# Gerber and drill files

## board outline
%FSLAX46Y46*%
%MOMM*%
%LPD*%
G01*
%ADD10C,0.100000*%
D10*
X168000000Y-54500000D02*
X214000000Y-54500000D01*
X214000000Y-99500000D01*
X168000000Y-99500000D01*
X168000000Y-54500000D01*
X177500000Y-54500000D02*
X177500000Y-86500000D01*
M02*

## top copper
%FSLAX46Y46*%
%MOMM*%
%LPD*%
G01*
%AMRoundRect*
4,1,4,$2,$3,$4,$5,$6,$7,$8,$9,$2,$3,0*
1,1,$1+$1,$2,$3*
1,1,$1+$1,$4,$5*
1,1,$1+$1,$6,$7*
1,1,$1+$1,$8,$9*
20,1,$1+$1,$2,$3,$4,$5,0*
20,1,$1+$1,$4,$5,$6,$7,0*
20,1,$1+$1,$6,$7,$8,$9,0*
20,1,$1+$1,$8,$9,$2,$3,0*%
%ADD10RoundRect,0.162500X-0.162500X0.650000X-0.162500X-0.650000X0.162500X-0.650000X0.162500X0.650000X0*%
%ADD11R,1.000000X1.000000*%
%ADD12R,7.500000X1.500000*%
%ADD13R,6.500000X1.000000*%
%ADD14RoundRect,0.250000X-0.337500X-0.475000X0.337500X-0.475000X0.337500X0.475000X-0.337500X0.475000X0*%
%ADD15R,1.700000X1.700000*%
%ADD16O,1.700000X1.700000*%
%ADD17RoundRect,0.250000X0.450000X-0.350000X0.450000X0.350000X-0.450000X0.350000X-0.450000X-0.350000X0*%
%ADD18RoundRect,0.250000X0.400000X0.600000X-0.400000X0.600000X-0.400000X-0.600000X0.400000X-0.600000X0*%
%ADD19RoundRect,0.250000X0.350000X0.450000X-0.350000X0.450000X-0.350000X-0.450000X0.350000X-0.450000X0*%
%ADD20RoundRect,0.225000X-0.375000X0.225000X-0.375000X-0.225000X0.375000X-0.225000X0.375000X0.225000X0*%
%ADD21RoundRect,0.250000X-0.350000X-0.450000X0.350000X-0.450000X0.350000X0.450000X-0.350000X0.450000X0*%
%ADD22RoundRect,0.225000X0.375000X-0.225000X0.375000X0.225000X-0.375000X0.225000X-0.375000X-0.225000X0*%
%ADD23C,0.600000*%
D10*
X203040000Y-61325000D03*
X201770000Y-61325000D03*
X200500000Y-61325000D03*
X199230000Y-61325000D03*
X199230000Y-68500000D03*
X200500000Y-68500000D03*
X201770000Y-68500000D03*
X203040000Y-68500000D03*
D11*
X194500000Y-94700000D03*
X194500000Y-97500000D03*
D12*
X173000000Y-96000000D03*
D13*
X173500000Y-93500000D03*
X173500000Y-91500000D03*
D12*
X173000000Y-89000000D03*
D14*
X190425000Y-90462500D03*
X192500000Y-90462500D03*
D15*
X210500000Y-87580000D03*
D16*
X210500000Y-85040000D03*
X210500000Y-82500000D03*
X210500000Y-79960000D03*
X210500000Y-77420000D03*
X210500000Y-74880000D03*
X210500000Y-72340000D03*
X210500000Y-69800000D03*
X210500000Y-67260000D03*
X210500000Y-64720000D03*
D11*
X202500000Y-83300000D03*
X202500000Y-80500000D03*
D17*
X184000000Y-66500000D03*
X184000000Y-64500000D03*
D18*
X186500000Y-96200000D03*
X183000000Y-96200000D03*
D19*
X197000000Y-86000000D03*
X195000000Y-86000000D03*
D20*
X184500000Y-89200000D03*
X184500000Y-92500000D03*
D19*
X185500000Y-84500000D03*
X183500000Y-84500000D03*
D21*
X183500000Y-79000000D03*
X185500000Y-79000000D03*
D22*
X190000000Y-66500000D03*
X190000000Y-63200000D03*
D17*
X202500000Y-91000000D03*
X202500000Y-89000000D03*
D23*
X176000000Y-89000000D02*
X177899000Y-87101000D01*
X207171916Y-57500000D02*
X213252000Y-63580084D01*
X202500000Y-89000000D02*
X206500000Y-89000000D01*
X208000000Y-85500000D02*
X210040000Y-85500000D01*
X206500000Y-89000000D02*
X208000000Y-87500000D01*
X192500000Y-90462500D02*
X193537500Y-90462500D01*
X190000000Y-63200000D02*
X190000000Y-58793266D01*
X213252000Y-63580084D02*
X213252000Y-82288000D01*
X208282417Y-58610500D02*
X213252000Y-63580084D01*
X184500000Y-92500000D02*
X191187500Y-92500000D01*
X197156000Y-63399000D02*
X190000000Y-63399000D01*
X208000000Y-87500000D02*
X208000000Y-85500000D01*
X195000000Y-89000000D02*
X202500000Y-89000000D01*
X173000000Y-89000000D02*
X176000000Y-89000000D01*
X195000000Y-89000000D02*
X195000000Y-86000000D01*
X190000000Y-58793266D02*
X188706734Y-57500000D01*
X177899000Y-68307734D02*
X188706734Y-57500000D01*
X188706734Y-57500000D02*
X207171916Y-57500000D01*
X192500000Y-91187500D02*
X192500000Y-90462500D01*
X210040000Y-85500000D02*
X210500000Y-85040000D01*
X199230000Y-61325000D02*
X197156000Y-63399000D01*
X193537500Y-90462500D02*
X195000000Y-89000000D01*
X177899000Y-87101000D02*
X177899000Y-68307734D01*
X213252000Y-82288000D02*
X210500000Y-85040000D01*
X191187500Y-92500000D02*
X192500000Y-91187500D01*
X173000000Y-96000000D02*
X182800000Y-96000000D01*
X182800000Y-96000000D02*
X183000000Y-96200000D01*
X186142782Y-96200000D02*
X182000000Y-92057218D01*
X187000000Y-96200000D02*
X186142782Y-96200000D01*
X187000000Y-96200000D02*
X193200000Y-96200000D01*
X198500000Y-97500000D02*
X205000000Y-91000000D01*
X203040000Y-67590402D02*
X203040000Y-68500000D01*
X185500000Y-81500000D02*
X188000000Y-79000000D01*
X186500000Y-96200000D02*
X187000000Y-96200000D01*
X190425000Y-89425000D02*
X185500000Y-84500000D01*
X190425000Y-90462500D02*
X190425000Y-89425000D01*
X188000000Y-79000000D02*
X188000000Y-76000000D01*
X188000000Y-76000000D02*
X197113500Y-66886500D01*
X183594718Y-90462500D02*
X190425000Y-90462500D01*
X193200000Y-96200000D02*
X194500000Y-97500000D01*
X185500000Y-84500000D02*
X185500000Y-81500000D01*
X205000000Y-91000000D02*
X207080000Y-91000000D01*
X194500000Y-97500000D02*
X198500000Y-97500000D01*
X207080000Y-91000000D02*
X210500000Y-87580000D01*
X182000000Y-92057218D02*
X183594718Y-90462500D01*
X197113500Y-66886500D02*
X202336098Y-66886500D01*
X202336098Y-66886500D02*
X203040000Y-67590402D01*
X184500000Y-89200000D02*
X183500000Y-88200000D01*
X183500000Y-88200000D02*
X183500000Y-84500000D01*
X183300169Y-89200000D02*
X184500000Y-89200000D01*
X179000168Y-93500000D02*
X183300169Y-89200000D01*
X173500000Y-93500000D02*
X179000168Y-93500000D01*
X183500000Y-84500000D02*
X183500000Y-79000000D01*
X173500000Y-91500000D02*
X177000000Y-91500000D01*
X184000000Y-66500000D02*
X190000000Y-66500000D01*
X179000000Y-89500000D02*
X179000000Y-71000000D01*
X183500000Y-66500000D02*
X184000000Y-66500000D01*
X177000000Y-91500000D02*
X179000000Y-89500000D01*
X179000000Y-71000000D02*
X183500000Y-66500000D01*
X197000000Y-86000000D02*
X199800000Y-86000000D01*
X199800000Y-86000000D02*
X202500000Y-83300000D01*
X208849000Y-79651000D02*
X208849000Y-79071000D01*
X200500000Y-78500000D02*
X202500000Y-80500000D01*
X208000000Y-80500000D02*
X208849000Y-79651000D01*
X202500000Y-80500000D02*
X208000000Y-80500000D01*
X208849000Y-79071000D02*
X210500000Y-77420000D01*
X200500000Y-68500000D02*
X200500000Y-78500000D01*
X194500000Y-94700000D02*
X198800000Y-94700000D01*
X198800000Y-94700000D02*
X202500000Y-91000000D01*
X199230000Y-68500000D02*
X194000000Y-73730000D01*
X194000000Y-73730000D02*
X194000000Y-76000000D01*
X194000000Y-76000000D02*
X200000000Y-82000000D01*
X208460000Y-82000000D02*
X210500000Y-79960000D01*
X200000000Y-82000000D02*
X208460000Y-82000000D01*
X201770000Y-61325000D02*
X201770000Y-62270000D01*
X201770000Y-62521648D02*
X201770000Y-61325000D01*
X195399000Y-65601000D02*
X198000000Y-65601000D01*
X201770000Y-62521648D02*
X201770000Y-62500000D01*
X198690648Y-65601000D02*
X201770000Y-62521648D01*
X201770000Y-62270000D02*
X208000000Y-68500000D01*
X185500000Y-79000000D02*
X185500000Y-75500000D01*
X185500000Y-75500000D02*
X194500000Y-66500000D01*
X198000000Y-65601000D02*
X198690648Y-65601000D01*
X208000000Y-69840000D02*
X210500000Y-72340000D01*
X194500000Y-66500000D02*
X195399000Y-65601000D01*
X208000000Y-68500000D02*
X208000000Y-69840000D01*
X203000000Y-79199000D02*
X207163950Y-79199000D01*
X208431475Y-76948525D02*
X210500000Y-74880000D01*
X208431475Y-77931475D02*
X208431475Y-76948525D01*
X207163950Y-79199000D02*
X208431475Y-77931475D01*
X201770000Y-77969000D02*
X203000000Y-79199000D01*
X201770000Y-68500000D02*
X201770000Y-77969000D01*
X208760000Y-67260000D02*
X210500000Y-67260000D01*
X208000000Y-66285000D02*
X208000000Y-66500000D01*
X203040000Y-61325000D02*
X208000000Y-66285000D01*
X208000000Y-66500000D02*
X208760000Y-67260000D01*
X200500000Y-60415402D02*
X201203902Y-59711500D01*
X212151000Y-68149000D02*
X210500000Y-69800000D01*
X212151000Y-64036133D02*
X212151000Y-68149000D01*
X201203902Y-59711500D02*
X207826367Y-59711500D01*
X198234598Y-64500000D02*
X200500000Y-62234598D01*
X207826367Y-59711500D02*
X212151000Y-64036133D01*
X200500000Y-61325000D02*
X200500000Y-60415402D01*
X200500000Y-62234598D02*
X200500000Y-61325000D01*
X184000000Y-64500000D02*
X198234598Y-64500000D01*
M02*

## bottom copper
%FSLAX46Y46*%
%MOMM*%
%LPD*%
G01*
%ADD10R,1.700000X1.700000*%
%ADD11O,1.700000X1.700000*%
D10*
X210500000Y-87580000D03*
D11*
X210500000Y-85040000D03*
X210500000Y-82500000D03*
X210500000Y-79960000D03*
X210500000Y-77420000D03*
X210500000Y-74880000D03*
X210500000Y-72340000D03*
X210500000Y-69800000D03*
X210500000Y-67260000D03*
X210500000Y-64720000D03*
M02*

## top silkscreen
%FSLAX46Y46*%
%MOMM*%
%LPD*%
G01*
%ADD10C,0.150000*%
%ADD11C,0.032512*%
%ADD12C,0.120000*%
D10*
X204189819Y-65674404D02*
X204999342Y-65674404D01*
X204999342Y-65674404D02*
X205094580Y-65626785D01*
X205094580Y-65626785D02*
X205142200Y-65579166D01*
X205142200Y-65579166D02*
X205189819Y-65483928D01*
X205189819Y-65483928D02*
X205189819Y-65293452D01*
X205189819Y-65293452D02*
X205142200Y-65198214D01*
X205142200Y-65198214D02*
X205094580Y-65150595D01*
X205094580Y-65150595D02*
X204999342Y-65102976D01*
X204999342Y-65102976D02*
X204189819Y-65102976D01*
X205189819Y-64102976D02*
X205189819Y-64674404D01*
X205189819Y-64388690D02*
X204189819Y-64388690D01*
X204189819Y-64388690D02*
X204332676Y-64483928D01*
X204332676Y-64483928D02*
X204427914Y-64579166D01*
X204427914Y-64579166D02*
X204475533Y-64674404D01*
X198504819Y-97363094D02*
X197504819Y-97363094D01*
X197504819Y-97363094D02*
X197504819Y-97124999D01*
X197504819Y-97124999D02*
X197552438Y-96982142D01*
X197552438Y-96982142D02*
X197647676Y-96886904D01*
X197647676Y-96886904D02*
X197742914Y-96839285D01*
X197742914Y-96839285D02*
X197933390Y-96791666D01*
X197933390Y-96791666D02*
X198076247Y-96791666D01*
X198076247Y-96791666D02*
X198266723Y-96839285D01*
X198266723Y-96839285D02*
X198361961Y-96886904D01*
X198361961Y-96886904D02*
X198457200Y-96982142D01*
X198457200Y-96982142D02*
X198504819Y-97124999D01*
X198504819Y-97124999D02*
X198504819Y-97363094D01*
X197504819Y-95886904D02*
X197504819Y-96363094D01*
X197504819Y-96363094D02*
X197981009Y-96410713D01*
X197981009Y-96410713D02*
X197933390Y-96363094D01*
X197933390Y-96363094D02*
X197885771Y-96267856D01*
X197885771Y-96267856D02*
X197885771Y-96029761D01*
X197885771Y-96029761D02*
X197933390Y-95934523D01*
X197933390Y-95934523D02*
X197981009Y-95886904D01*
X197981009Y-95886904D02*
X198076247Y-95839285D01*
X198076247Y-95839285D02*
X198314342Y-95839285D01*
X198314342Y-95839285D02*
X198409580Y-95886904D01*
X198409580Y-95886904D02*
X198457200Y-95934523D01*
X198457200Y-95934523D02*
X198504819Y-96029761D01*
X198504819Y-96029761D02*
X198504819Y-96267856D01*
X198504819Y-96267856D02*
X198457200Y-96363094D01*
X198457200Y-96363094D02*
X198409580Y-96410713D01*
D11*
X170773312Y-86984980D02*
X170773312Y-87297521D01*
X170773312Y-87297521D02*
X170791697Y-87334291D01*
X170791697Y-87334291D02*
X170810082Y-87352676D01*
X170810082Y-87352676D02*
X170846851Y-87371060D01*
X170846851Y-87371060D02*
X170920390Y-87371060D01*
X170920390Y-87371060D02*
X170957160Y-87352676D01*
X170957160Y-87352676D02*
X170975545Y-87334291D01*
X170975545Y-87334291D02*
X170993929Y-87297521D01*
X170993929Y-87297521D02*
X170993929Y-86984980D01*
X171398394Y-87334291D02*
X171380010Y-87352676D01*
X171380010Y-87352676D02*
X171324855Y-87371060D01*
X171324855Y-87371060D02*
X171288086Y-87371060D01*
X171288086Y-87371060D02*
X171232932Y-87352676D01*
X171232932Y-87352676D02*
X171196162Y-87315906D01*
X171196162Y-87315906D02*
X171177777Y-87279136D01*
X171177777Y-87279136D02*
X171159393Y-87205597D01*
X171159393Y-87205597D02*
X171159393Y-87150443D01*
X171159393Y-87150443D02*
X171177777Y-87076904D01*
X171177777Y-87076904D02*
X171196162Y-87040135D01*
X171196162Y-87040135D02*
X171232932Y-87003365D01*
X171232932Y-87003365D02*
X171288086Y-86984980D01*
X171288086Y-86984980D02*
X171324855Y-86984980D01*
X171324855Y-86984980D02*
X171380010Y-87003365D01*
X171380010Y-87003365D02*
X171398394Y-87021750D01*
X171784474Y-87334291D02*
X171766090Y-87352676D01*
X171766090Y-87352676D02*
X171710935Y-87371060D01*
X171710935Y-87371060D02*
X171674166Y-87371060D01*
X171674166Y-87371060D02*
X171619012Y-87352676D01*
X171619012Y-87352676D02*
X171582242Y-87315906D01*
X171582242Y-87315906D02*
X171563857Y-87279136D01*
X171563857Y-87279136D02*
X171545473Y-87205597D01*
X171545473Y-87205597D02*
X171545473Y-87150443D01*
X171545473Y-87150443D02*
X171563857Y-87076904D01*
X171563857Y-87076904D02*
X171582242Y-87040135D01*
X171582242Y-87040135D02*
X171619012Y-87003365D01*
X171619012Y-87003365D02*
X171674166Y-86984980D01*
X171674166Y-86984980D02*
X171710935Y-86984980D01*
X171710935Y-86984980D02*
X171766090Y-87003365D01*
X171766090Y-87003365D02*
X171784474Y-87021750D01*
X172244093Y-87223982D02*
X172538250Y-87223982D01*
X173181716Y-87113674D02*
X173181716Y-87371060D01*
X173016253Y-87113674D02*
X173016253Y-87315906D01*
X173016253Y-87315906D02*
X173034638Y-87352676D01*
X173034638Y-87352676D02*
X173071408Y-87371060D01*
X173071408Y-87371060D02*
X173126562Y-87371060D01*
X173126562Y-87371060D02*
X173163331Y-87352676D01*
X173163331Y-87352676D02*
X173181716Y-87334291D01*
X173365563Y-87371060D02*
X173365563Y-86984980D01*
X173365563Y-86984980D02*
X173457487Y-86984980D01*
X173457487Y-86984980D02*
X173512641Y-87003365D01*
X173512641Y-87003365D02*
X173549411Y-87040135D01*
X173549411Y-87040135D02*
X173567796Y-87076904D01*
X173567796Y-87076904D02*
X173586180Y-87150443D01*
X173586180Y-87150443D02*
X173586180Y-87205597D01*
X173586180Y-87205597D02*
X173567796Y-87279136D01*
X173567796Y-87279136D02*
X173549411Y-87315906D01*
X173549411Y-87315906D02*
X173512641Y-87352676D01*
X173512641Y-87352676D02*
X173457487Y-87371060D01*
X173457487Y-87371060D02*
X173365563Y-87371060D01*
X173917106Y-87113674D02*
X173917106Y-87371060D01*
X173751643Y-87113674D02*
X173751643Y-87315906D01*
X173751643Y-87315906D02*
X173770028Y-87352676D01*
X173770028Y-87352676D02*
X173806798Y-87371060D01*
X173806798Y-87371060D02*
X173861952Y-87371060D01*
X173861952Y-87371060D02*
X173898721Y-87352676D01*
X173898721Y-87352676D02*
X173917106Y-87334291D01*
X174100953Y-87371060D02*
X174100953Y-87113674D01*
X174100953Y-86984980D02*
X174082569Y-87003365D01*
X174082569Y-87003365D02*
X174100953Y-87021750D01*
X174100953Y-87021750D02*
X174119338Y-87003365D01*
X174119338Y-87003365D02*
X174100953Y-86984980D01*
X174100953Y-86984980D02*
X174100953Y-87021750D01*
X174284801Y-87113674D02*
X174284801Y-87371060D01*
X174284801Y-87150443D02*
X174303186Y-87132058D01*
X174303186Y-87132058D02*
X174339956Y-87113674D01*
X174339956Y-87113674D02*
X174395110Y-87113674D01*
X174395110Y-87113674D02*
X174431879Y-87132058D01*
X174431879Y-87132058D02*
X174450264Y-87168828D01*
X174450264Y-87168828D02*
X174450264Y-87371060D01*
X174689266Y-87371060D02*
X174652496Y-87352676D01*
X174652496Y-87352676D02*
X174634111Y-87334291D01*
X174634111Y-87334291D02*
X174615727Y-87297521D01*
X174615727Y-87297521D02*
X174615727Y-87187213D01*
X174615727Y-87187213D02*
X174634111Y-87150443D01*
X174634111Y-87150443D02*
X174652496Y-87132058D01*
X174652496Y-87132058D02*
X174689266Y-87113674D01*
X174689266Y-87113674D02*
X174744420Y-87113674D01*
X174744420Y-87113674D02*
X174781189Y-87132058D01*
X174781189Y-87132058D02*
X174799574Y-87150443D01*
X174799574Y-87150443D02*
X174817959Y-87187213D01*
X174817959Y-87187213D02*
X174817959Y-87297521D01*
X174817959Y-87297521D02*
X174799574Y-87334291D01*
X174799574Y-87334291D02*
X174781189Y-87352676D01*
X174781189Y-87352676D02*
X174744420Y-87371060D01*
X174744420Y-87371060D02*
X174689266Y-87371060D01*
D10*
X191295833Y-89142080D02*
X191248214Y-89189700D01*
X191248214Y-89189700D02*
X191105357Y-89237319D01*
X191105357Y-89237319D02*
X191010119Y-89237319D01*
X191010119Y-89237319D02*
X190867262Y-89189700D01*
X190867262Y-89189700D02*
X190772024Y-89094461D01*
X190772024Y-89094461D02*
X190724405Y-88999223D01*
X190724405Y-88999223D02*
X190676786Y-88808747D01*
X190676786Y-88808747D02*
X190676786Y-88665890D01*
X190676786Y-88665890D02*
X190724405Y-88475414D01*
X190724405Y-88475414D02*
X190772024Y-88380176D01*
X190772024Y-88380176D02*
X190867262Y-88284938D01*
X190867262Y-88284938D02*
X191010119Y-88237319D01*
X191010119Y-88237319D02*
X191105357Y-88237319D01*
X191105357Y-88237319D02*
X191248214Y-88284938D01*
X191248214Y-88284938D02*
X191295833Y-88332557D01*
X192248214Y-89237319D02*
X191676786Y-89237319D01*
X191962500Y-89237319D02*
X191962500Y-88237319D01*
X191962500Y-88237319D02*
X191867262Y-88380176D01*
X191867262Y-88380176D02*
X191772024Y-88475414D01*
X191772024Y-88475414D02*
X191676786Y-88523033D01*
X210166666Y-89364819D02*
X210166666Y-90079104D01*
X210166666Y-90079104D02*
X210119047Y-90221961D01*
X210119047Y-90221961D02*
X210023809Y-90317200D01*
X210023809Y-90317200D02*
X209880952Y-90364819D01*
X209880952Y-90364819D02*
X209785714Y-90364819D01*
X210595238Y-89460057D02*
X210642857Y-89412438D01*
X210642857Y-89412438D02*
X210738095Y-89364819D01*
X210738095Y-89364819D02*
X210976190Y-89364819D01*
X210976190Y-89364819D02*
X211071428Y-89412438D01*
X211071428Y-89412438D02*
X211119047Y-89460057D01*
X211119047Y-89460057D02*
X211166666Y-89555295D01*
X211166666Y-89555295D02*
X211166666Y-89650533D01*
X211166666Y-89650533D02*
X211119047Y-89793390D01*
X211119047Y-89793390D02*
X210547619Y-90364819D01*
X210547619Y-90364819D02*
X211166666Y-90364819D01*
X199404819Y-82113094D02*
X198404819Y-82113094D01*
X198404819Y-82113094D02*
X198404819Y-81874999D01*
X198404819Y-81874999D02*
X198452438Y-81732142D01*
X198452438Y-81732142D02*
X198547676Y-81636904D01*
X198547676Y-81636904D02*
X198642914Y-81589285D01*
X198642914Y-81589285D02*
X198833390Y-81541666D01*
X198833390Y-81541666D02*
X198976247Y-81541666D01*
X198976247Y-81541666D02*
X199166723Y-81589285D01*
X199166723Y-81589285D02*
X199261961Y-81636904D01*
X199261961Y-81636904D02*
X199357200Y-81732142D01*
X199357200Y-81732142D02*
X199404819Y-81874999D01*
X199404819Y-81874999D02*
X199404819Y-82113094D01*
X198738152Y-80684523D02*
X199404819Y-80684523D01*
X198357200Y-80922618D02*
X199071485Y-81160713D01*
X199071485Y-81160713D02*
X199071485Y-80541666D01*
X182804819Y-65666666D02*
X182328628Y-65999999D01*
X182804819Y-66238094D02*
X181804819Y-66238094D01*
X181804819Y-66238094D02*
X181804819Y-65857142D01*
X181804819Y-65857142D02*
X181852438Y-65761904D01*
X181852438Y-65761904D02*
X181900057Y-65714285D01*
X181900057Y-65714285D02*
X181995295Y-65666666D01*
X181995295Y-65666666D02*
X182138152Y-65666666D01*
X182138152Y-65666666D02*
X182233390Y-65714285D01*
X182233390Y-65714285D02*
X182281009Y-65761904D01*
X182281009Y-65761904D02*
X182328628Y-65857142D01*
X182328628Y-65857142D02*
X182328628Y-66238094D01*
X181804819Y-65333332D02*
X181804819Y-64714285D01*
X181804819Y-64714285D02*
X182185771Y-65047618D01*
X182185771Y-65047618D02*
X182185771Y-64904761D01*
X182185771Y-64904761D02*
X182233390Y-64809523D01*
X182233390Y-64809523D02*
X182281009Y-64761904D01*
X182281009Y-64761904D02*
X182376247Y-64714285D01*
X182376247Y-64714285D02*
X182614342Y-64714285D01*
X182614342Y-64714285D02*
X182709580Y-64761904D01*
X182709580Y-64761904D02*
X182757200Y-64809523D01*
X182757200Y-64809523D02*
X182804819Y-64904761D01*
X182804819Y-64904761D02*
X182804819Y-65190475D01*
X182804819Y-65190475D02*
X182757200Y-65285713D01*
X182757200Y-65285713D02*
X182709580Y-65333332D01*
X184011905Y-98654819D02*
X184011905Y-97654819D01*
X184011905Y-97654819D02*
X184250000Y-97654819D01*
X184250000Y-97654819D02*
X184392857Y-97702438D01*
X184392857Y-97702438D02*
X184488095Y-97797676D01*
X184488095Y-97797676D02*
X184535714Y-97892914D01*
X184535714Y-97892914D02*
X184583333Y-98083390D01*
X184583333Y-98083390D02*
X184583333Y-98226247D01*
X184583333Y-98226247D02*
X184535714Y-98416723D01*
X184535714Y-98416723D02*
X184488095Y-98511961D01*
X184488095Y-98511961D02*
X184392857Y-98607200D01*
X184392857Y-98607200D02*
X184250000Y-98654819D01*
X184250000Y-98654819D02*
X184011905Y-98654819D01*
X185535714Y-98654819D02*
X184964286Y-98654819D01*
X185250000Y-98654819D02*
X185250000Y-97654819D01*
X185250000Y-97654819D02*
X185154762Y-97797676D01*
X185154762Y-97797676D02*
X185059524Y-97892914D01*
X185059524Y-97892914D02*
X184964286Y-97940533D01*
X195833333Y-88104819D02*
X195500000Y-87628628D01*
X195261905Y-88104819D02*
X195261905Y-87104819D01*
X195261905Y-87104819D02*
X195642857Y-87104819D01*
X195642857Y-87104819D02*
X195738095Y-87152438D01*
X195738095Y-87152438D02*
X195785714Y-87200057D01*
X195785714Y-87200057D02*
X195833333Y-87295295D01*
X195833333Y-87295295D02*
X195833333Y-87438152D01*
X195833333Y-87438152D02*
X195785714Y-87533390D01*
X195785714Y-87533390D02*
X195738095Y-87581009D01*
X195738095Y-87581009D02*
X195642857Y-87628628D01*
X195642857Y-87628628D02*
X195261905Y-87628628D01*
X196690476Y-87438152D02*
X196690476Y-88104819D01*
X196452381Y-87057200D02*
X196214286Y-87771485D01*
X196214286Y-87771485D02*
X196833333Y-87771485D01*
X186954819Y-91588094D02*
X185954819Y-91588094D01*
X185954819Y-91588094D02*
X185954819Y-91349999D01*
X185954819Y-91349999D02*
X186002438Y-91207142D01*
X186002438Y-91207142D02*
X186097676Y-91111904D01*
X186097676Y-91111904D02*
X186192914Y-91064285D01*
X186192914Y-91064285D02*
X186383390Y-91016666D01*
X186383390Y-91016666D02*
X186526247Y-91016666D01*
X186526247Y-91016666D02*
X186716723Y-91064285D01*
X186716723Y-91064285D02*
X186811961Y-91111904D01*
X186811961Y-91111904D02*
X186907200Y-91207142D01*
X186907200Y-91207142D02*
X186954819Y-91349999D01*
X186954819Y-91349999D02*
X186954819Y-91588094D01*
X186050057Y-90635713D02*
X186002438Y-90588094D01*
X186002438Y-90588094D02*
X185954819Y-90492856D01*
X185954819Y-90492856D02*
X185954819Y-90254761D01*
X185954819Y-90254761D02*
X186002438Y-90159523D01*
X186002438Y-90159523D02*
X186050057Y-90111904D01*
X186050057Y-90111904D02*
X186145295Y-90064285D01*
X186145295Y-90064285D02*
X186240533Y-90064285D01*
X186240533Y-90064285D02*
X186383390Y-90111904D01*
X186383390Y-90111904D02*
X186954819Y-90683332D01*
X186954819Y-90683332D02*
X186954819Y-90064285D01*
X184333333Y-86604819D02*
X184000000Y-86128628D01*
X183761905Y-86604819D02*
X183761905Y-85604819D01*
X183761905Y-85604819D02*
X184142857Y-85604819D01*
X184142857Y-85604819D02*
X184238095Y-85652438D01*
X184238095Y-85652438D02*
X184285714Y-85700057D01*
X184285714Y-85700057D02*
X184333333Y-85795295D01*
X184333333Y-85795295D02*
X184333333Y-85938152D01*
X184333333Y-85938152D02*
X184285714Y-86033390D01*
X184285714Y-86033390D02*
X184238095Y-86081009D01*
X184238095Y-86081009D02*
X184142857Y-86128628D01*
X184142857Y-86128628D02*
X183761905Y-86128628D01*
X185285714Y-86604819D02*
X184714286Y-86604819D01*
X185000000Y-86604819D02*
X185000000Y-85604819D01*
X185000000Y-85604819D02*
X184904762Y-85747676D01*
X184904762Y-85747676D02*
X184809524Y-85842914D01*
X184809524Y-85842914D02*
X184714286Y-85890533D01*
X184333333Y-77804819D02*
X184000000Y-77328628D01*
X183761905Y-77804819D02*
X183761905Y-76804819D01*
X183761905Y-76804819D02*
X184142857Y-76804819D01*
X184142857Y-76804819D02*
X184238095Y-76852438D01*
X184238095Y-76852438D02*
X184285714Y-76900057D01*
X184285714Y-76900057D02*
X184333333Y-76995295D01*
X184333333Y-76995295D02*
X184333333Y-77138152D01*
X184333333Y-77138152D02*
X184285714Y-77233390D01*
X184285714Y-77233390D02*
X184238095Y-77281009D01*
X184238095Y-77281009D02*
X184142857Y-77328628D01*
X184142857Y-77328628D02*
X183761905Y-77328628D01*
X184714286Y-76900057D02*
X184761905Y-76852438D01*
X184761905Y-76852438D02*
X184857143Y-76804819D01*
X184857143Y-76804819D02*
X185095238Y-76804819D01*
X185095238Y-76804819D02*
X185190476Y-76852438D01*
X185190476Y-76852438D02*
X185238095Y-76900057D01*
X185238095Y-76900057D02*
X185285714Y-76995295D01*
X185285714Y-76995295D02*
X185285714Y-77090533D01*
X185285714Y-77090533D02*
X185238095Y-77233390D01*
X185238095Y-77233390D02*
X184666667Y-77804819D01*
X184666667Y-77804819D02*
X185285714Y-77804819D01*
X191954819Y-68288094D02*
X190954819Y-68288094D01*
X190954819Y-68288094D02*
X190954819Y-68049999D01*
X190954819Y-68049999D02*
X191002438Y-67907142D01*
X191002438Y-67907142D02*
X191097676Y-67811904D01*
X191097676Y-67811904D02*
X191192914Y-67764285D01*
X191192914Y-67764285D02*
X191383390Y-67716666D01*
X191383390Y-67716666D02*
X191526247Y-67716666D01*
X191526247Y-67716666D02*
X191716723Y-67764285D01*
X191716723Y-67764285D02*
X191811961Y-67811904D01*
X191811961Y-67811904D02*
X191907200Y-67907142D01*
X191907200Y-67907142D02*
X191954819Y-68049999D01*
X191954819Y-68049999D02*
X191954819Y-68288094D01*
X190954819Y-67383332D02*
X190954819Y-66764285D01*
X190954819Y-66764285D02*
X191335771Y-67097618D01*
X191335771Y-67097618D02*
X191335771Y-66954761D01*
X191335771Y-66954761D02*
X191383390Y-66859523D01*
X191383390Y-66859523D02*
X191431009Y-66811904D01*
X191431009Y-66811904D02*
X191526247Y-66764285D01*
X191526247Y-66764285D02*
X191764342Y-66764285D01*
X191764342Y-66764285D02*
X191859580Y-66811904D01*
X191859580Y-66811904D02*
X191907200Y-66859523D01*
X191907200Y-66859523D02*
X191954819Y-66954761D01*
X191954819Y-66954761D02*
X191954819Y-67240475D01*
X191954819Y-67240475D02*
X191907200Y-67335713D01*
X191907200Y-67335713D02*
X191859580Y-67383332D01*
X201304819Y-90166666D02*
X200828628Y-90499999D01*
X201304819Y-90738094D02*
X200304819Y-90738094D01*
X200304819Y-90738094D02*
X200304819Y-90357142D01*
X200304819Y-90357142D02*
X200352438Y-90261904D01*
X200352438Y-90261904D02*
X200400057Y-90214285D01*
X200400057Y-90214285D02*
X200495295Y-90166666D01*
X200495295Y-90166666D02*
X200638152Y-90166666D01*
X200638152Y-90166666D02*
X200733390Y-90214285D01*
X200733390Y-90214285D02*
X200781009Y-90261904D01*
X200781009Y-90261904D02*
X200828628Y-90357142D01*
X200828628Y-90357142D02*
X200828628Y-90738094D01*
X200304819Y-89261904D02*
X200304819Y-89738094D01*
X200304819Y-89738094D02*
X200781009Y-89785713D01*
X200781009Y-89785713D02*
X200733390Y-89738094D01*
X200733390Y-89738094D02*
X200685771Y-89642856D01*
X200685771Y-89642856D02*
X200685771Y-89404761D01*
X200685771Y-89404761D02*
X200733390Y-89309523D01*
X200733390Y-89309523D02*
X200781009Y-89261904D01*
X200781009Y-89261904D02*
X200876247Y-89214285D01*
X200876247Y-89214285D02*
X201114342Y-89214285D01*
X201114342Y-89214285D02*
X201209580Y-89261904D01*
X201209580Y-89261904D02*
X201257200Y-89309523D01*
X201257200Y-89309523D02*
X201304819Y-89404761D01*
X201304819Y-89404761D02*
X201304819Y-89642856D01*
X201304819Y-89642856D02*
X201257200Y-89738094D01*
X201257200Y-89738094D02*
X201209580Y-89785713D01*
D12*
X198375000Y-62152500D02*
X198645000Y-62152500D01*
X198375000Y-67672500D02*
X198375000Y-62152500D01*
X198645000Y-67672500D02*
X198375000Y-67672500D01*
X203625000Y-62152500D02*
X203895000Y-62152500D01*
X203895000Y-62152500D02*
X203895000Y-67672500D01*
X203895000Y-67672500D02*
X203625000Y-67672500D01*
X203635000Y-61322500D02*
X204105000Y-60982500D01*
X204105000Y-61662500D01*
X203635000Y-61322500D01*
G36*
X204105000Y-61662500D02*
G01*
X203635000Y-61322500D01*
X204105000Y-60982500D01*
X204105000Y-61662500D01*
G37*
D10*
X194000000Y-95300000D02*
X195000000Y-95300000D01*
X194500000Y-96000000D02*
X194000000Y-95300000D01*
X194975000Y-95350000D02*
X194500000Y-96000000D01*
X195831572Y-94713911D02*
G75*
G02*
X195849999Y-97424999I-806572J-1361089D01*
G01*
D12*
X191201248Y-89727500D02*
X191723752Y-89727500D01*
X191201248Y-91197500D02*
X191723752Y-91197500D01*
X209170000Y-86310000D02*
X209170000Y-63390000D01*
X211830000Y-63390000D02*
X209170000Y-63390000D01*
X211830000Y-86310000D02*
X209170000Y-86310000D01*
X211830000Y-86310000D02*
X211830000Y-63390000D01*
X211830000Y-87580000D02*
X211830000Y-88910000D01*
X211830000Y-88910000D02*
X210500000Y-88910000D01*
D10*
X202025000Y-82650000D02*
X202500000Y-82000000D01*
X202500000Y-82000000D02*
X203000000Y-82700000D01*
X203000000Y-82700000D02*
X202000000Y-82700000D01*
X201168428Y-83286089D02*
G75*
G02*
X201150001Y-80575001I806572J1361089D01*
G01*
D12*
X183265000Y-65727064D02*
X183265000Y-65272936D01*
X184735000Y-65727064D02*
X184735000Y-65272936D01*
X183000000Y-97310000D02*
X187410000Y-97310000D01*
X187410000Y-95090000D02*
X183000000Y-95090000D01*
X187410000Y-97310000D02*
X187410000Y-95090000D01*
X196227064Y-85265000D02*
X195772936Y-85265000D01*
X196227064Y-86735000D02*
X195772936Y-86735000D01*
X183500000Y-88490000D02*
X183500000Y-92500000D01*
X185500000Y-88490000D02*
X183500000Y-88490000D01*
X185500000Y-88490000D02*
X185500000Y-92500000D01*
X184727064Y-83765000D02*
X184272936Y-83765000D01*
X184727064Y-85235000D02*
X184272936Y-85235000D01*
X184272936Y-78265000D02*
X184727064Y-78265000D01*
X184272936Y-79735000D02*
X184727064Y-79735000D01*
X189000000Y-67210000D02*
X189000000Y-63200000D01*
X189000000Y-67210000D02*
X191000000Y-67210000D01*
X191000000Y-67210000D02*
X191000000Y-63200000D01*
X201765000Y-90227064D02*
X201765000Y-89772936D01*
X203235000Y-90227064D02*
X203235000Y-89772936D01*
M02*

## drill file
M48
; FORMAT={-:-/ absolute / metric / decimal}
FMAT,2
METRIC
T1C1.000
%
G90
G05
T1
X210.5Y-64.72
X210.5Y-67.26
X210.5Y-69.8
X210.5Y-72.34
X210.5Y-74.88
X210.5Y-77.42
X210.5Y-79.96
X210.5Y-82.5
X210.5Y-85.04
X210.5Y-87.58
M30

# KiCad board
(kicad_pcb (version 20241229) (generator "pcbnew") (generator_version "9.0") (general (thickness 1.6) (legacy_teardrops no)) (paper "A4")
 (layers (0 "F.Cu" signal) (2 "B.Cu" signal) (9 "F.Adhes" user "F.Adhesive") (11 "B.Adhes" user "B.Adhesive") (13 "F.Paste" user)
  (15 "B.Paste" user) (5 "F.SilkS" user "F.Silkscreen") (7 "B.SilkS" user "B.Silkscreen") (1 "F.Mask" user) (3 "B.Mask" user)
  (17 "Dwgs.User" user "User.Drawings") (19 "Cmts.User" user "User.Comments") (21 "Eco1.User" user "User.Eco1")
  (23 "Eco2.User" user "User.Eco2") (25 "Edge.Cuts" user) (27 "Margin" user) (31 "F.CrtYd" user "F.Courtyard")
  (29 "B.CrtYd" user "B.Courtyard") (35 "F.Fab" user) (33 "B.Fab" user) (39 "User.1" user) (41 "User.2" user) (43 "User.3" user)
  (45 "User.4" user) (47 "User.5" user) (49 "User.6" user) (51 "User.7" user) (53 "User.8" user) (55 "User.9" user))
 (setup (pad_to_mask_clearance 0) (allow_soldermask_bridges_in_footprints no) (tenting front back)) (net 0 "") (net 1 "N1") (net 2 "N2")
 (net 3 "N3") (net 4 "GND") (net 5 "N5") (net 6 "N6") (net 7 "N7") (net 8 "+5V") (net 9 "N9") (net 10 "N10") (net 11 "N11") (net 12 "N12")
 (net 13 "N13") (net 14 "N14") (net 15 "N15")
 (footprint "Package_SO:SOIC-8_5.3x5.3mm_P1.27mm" (layer "F.Cu") (at 201.135 64.9125 -90)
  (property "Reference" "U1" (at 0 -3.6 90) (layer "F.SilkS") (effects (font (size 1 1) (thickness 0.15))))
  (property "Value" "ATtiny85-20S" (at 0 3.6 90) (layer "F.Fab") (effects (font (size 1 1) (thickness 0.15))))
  (fp_line (start -2.76 2.76) (end -2.76 2.49) (stroke (width 0.12) (type solid)) (layer "F.SilkS"))
  (fp_line (start 2.76 2.76) (end -2.76 2.76) (stroke (width 0.12) (type solid)) (layer "F.SilkS"))
  (fp_line (start 2.76 2.49) (end 2.76 2.76) (stroke (width 0.12) (type solid)) (layer "F.SilkS"))
  (fp_line (start -2.76 -2.49) (end -2.76 -2.76) (stroke (width 0.12) (type solid)) (layer "F.SilkS"))
  (fp_line (start -2.76 -2.76) (end 2.76 -2.76) (stroke (width 0.12) (type solid)) (layer "F.SilkS"))
  (fp_line (start 2.76 -2.76) (end 2.76 -2.49) (stroke (width 0.12) (type solid)) (layer "F.SilkS"))
  (fp_poly (pts (xy -3.59 -2.5) (xy -3.93 -2.97) (xy -3.25 -2.97)) (stroke (width 0.12) (type solid)) (fill yes) (layer "F.SilkS"))
  (pad "1" smd roundrect (at -3.5875 -1.905 270) (size 1.625 0.65) (layers "F.Cu" "F.Mask" "F.Paste") (roundrect_rratio 0.25) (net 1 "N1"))
  (pad "2" smd roundrect (at -3.5875 -0.635 270) (size 1.625 0.65) (layers "F.Cu" "F.Mask" "F.Paste") (roundrect_rratio 0.25) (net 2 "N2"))
  (pad "3" smd roundrect (at -3.5875 0.635 270) (size 1.625 0.65) (layers "F.Cu" "F.Mask" "F.Paste") (roundrect_rratio 0.25) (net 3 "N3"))
  (pad "4" smd roundrect (at -3.5875 1.905 270) (size 1.625 0.65) (layers "F.Cu" "F.Mask" "F.Paste") (roundrect_rratio 0.25) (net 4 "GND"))
  (pad "5" smd roundrect (at 3.5875 1.905 270) (size 1.625 0.65) (layers "F.Cu" "F.Mask" "F.Paste") (roundrect_rratio 0.25) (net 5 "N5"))
  (pad "6" smd roundrect (at 3.5875 0.635 270) (size 1.625 0.65) (layers "F.Cu" "F.Mask" "F.Paste") (roundrect_rratio 0.25) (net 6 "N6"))
  (pad "7" smd roundrect (at 3.5875 -0.635 270) (size 1.625 0.65) (layers "F.Cu" "F.Mask" "F.Paste") (roundrect_rratio 0.25) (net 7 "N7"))
  (pad "8" smd roundrect (at 3.5875 -1.905 270) (size 1.625 0.65) (layers "F.Cu" "F.Mask" "F.Paste") (roundrect_rratio 0.25) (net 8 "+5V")))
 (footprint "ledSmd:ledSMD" (layer "F.Cu") (at 194.5 96.5 -90)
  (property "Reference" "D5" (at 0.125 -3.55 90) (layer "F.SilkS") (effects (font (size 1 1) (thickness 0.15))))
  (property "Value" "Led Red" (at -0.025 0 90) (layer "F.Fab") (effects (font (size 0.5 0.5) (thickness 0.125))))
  (fp_line (start -1.2 0.5) (end -1.2 -0.5) (stroke (width 0.15) (type solid)) (layer "F.SilkS"))
  (fp_line (start -0.5 0) (end -1.2 0.5) (stroke (width 0.15) (type solid)) (layer "F.SilkS"))
  (fp_line (start -1.15 -0.475) (end -0.5 0) (stroke (width 0.15) (type solid)) (layer "F.SilkS"))
  (fp_arc (start -1.786089 -1.331572) (mid -0.435753 -2.107089) (end 0.924999 -1.349999) (stroke (width 0.15) (type solid))
   (layer "F.SilkS"))
  (pad "1" smd rect (at -1.8 0 270) (size 1 1) (layers "F.Cu" "F.Mask" "F.Paste") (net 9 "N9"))
  (pad "2" smd rect (at 1 0 270) (size 1 1) (layers "F.Cu" "F.Mask" "F.Paste") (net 8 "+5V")))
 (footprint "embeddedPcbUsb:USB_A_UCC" (layer "F.Cu") (at 173.2 92.5)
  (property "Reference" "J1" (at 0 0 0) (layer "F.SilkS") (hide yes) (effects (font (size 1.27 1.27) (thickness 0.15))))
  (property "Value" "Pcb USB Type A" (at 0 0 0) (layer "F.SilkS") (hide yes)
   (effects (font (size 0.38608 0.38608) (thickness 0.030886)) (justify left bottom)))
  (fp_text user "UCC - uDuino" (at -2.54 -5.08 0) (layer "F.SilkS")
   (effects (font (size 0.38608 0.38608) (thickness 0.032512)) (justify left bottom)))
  (pad "1" smd rect (at -0.2 3.5) (size 7.5 1.5) (layers "F.Cu" "F.Mask" "F.Paste") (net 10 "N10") (solder_mask_margin 0.1016))
  (pad "2" smd rect (at 0.3 1) (size 6.5 1) (layers "F.Cu" "F.Mask" "F.Paste") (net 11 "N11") (solder_mask_margin 0.1016))
  (pad "3" smd rect (at 0.3 -1) (size 6.5 1) (layers "F.Cu" "F.Mask" "F.Paste") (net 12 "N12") (solder_mask_margin 0.1016))
  (pad "4" smd rect (at -0.2 -3.5) (size 7.5 1.5) (layers "F.Cu" "F.Mask" "F.Paste") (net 4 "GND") (solder_mask_margin 0.1016)))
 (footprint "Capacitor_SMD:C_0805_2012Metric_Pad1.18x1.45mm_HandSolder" (layer "F.Cu") (at 191.4625 90.4625)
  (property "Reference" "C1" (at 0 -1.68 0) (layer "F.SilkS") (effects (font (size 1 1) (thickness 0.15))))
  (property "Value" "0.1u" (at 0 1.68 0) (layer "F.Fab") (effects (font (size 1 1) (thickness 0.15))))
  (fp_line (start -0.261252 -0.735) (end 0.261252 -0.735) (stroke (width 0.12) (type solid)) (layer "F.SilkS"))
  (fp_line (start -0.261252 0.735) (end 0.261252 0.735) (stroke (width 0.12) (type solid)) (layer "F.SilkS"))
  (pad "1" smd roundrect (at -1.0375 0) (size 1.175 1.45) (layers "F.Cu" "F.Mask" "F.Paste") (roundrect_rratio 0.212766) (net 8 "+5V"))
  (pad "2" smd roundrect (at 1.0375 0) (size 1.175 1.45) (layers "F.Cu" "F.Mask" "F.Paste") (roundrect_rratio 0.212766) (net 4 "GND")))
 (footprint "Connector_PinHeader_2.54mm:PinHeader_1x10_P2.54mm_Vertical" (layer "F.Cu") (at 210.5 87.58 180)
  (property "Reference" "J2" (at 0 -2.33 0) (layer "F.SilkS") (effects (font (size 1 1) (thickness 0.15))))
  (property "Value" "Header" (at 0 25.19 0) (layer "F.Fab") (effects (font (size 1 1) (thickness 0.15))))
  (fp_line (start 1.33 1.27) (end 1.33 24.19) (stroke (width 0.12) (type solid)) (layer "F.SilkS"))
  (fp_line (start -1.33 24.19) (end 1.33 24.19) (stroke (width 0.12) (type solid)) (layer "F.SilkS"))
  (fp_line (start -1.33 1.27) (end 1.33 1.27) (stroke (width 0.12) (type solid)) (layer "F.SilkS"))
  (fp_line (start -1.33 1.27) (end -1.33 24.19) (stroke (width 0.12) (type solid)) (layer "F.SilkS"))
  (fp_line (start -1.33 0) (end -1.33 -1.33) (stroke (width 0.12) (type solid)) (layer "F.SilkS"))
  (fp_line (start -1.33 -1.33) (end 0 -1.33) (stroke (width 0.12) (type solid)) (layer "F.SilkS"))
  (pad "1" thru_hole rect (at 0 0 180) (size 1.7 1.7) (drill 1) (layers "*.Cu" "*.Mask") (remove_unused_layers no) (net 8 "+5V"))
  (pad "2" thru_hole oval (at 0 2.54 180) (size 1.7 1.7) (drill 1) (layers "*.Cu" "*.Mask") (remove_unused_layers no) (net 4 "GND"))
  (pad "3" thru_hole oval (at 0 5.08 180) (size 1.7 1.7) (drill 1) (layers "*.Cu" "*.Mask") (remove_unused_layers no) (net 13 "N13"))
  (pad "4" thru_hole oval (at 0 7.62 180) (size 1.7 1.7) (drill 1) (layers "*.Cu" "*.Mask") (remove_unused_layers no) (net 5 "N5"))
  (pad "5" thru_hole oval (at 0 10.16 180) (size 1.7 1.7) (drill 1) (layers "*.Cu" "*.Mask") (remove_unused_layers no) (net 6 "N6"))
  (pad "6" thru_hole oval (at 0 12.7 180) (size 1.7 1.7) (drill 1) (layers "*.Cu" "*.Mask") (remove_unused_layers no) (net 7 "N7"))
  (pad "7" thru_hole oval (at 0 15.24 180) (size 1.7 1.7) (drill 1) (layers "*.Cu" "*.Mask") (remove_unused_layers no) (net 2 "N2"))
  (pad "8" thru_hole oval (at 0 17.78 180) (size 1.7 1.7) (drill 1) (layers "*.Cu" "*.Mask") (remove_unused_layers no) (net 3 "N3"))
  (pad "9" thru_hole oval (at 0 20.32 180) (size 1.7 1.7) (drill 1) (layers "*.Cu" "*.Mask") (remove_unused_layers no) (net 1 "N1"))
  (pad "10" thru_hole oval (at 0 22.86 180) (size 1.7 1.7) (drill 1) (layers "*.Cu" "*.Mask") (remove_unused_layers no) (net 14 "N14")))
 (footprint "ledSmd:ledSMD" (layer "F.Cu") (at 202.5 81.5 90)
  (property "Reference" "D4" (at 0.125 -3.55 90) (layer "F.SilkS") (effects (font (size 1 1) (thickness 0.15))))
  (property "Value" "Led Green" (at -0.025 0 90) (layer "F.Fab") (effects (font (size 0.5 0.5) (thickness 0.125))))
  (fp_line (start -1.15 -0.475) (end -0.5 0) (stroke (width 0.15) (type solid)) (layer "F.SilkS"))
  (fp_line (start -0.5 0) (end -1.2 0.5) (stroke (width 0.15) (type solid)) (layer "F.SilkS"))
  (fp_line (start -1.2 0.5) (end -1.2 -0.5) (stroke (width 0.15) (type solid)) (layer "F.SilkS"))
  (fp_arc (start -1.786089 -1.331572) (mid -0.435753 -2.107089) (end 0.924999 -1.349999) (stroke (width 0.15) (type solid))
   (layer "F.SilkS"))
  (pad "1" smd rect (at -1.8 0 90) (size 1 1) (layers "F.Cu" "F.Mask" "F.Paste") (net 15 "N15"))
  (pad "2" smd rect (at 1 0 90) (size 1 1) (layers "F.Cu" "F.Mask" "F.Paste") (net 6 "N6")))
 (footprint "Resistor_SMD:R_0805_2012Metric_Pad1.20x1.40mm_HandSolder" (layer "F.Cu") (at 184 65.5 90)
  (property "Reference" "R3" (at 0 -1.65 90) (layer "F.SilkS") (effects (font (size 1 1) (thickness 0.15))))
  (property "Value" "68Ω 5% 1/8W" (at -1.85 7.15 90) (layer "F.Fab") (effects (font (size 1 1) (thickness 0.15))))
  (fp_line (start -0.227064 -0.735) (end 0.227064 -0.735) (stroke (width 0.12) (type solid)) (layer "F.SilkS"))
  (fp_line (start -0.227064 0.735) (end 0.227064 0.735) (stroke (width 0.12) (type solid)) (layer "F.SilkS"))
  (pad "1" smd roundrect (at -1 0 90) (size 1.2 1.4) (layers "F.Cu" "F.Mask" "F.Paste") (roundrect_rratio 0.208333) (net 12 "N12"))
  (pad "2" smd roundrect (at 1 0 90) (size 1.2 1.4) (layers "F.Cu" "F.Mask" "F.Paste") (roundrect_rratio 0.208333) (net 3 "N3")))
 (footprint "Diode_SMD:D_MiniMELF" (layer "F.Cu") (at 184.75 96.2 180)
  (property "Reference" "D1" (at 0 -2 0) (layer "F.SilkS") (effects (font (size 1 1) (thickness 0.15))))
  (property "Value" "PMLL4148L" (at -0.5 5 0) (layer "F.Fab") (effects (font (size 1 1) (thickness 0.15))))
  (fp_line (start 1.75 -1.11) (end -2.66 -1.11) (stroke (width 0.12) (type solid)) (layer "F.SilkS"))
  (fp_line (start -2.66 1.11) (end 1.75 1.11) (stroke (width 0.12) (type solid)) (layer "F.SilkS"))
  (fp_line (start -2.66 -1.11) (end -2.66 1.11) (stroke (width 0.12) (type solid)) (layer "F.SilkS"))
  (pad "1" smd roundrect (at -1.75 0 180) (size 1.3 1.7) (layers "F.Cu" "F.Mask" "F.Paste") (roundrect_rratio 0.1923076923) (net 8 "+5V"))
  (pad "2" smd roundrect (at 1.75 0 180) (size 1.3 1.7) (layers "F.Cu" "F.Mask" "F.Paste") (roundrect_rratio 0.1923076923) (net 10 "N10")))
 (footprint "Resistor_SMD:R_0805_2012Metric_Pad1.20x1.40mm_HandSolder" (layer "F.Cu") (at 196 86 180)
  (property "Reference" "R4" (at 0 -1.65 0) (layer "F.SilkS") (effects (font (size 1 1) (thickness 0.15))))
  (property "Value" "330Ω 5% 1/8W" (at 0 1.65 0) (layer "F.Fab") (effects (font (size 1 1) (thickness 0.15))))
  (fp_line (start -0.227064 0.735) (end 0.227064 0.735) (stroke (width 0.12) (type solid)) (layer "F.SilkS"))
  (fp_line (start -0.227064 -0.735) (end 0.227064 -0.735) (stroke (width 0.12) (type solid)) (layer "F.SilkS"))
  (pad "1" smd roundrect (at -1 0 180) (size 1.2 1.4) (layers "F.Cu" "F.Mask" "F.Paste") (roundrect_rratio 0.208333) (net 15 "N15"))
  (pad "2" smd roundrect (at 1 0 180) (size 1.2 1.4) (layers "F.Cu" "F.Mask" "F.Paste") (roundrect_rratio 0.208333) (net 4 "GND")))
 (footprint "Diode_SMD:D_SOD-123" (layer "F.Cu") (at 184.5 90.85 -90)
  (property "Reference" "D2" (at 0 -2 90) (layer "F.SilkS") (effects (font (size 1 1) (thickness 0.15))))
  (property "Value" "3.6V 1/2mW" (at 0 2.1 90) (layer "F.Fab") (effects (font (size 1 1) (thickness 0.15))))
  (fp_line (start -2.36 1) (end 1.65 1) (stroke (width 0.12) (type solid)) (layer "F.SilkS"))
  (fp_line (start -2.36 -1) (end -2.36 1) (stroke (width 0.12) (type solid)) (layer "F.SilkS"))
  (fp_line (start -2.36 -1) (end 1.65 -1) (stroke (width 0.12) (type solid)) (layer "F.SilkS"))
  (pad "1" smd roundrect (at -1.65 0 270) (size 0.9 1.2) (layers "F.Cu" "F.Mask" "F.Paste") (roundrect_rratio 0.25) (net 11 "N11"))
  (pad "2" smd roundrect (at 1.65 0 270) (size 0.9 1.2) (layers "F.Cu" "F.Mask" "F.Paste") (roundrect_rratio 0.25) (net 4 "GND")))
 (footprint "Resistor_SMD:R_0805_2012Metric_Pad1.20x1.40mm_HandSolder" (layer "F.Cu") (at 184.5 84.5 180)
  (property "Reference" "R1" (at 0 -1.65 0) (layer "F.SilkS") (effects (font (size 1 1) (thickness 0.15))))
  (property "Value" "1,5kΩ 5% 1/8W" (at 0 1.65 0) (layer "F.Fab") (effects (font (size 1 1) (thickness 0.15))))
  (fp_line (start -0.227064 0.735) (end 0.227064 0.735) (stroke (width 0.12) (type solid)) (layer "F.SilkS"))
  (fp_line (start -0.227064 -0.735) (end 0.227064 -0.735) (stroke (width 0.12) (type solid)) (layer "F.SilkS"))
  (pad "1" smd roundrect (at -1 0 180) (size 1.2 1.4) (layers "F.Cu" "F.Mask" "F.Paste") (roundrect_rratio 0.208333) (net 8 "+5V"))
  (pad "2" smd roundrect (at 1 0 180) (size 1.2 1.4) (layers "F.Cu" "F.Mask" "F.Paste") (roundrect_rratio 0.208333) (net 11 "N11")))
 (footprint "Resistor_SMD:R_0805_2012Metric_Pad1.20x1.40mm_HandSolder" (layer "F.Cu") (at 184.5 79)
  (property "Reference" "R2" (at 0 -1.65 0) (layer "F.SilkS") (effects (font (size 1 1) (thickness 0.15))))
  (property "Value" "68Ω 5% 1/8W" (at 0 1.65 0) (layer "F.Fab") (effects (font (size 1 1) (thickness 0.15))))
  (fp_line (start -0.227064 -0.735) (end 0.227064 -0.735) (stroke (width 0.12) (type solid)) (layer "F.SilkS"))
  (fp_line (start -0.227064 0.735) (end 0.227064 0.735) (stroke (width 0.12) (type solid)) (layer "F.SilkS"))
  (pad "1" smd roundrect (at -1 0) (size 1.2 1.4) (layers "F.Cu" "F.Mask" "F.Paste") (roundrect_rratio 0.208333) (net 11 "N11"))
  (pad "2" smd roundrect (at 1 0) (size 1.2 1.4) (layers "F.Cu" "F.Mask" "F.Paste") (roundrect_rratio 0.208333) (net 2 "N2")))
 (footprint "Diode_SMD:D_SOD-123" (layer "F.Cu") (at 190 64.85 90)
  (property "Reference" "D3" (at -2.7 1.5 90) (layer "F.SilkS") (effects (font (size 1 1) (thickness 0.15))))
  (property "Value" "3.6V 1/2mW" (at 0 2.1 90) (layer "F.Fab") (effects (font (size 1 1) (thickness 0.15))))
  (fp_line (start -2.36 -1) (end 1.65 -1) (stroke (width 0.12) (type solid)) (layer "F.SilkS"))
  (fp_line (start -2.36 -1) (end -2.36 1) (stroke (width 0.12) (type solid)) (layer "F.SilkS"))
  (fp_line (start -2.36 1) (end 1.65 1) (stroke (width 0.12) (type solid)) (layer "F.SilkS"))
  (pad "1" smd roundrect (at -1.65 0 90) (size 0.9 1.2) (layers "F.Cu" "F.Mask" "F.Paste") (roundrect_rratio 0.25) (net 12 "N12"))
  (pad "2" smd roundrect (at 1.65 0 90) (size 0.9 1.2) (layers "F.Cu" "F.Mask" "F.Paste") (roundrect_rratio 0.25) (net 4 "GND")))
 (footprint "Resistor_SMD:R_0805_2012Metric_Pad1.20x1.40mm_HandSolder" (layer "F.Cu") (at 202.5 90 90)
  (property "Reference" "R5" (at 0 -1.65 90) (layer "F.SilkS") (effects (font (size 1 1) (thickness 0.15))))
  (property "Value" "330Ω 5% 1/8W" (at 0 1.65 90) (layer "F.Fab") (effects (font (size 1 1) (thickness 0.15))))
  (fp_line (start -0.227064 -0.735) (end 0.227064 -0.735) (stroke (width 0.12) (type solid)) (layer "F.SilkS"))
  (fp_line (start -0.227064 0.735) (end 0.227064 0.735) (stroke (width 0.12) (type solid)) (layer "F.SilkS"))
  (pad "1" smd roundrect (at -1 0 90) (size 1.2 1.4) (layers "F.Cu" "F.Mask" "F.Paste") (roundrect_rratio 0.208333) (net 9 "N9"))
  (pad "2" smd roundrect (at 1 0 90) (size 1.2 1.4) (layers "F.Cu" "F.Mask" "F.Paste") (roundrect_rratio 0.208333) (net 4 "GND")))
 (gr_rect (start 168 54.5) (end 214 99.5) (stroke (width 0.1) (type default)) (fill no) (layer "Edge.Cuts"))
 (gr_line (start 177.5 54.5) (end 177.5 86.5) (stroke (width 0.1) (type default)) (layer "Edge.Cuts"))
 (segment (start 176 89) (end 177.899 87.101) (width 0.6) (layer "F.Cu") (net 4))
 (segment (start 207.171916 57.5) (end 213.252 63.580084) (width 0.6) (layer "F.Cu") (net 4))
 (segment (start 202.5 89) (end 206.5 89) (width 0.6) (layer "F.Cu") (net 4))
 (segment (start 208 85.5) (end 210.04 85.5) (width 0.6) (layer "F.Cu") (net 4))
 (segment (start 206.5 89) (end 208 87.5) (width 0.6) (layer "F.Cu") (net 4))
 (segment (start 192.5 90.4625) (end 193.5375 90.4625) (width 0.6) (layer "F.Cu") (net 4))
 (segment (start 190 63.2) (end 190 58.793266) (width 0.6) (layer "F.Cu") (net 4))
 (segment (start 213.252 63.580084) (end 213.252 82.288) (width 0.6) (layer "F.Cu") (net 4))
 (segment (start 208.282417 58.6105) (end 213.252 63.580084) (width 0.6) (layer "F.Cu") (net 4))
 (segment (start 184.5 92.5) (end 191.1875 92.5) (width 0.6) (layer "F.Cu") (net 4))
 (segment (start 197.156 63.399) (end 190 63.399) (width 0.6) (layer "F.Cu") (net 4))
 (segment (start 208 87.5) (end 208 85.5) (width 0.6) (layer "F.Cu") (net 4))
 (segment (start 195 89) (end 202.5 89) (width 0.6) (layer "F.Cu") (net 4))
 (segment (start 173 89) (end 176 89) (width 0.6) (layer "F.Cu") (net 4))
 (segment (start 195 89) (end 195 86) (width 0.6) (layer "F.Cu") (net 4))
 (segment (start 190 58.793266) (end 188.706734 57.5) (width 0.6) (layer "F.Cu") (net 4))
 (segment (start 177.899 68.307734) (end 188.706734 57.5) (width 0.6) (layer "F.Cu") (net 4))
 (segment (start 188.706734 57.5) (end 207.171916 57.5) (width 0.6) (layer "F.Cu") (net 4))
 (segment (start 192.5 91.1875) (end 192.5 90.4625) (width 0.6) (layer "F.Cu") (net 4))
 (segment (start 210.04 85.5) (end 210.5 85.04) (width 0.6) (layer "F.Cu") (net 4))
 (segment (start 199.23 61.325) (end 197.156 63.399) (width 0.6) (layer "F.Cu") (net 4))
 (segment (start 193.5375 90.4625) (end 195 89) (width 0.6) (layer "F.Cu") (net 4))
 (segment (start 177.899 87.101) (end 177.899 68.307734) (width 0.6) (layer "F.Cu") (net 4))
 (segment (start 213.252 82.288) (end 210.5 85.04) (width 0.6) (layer "F.Cu") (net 4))
 (segment (start 191.1875 92.5) (end 192.5 91.1875) (width 0.6) (layer "F.Cu") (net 4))
 (segment (start 173 96) (end 182.8 96) (width 0.6) (layer "F.Cu") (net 10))
 (segment (start 182.8 96) (end 183 96.2) (width 0.6) (layer "F.Cu") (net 10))
 (segment (start 186.142782 96.2) (end 182 92.057218) (width 0.6) (layer "F.Cu") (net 8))
 (segment (start 187 96.2) (end 186.142782 96.2) (width 0.6) (layer "F.Cu") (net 8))
 (segment (start 187 96.2) (end 193.2 96.2) (width 0.6) (layer "F.Cu") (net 8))
 (segment (start 198.5 97.5) (end 205 91) (width 0.6) (layer "F.Cu") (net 8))
 (segment (start 203.04 67.590402) (end 203.04 68.5) (width 0.6) (layer "F.Cu") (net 8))
 (segment (start 185.5 81.5) (end 188 79) (width 0.6) (layer "F.Cu") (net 8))
 (segment (start 186.5 96.2) (end 187 96.2) (width 0.6) (layer "F.Cu") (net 8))
 (segment (start 190.425 89.425) (end 185.5 84.5) (width 0.6) (layer "F.Cu") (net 8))
 (segment (start 190.425 90.4625) (end 190.425 89.425) (width 0.6) (layer "F.Cu") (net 8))
 (segment (start 188 79) (end 188 76) (width 0.6) (layer "F.Cu") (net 8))
 (segment (start 188 76) (end 197.1135 66.8865) (width 0.6) (layer "F.Cu") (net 8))
 (segment (start 183.594718 90.4625) (end 190.425 90.4625) (width 0.6) (layer "F.Cu") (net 8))
 (segment (start 193.2 96.2) (end 194.5 97.5) (width 0.6) (layer "F.Cu") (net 8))
 (segment (start 185.5 84.5) (end 185.5 81.5) (width 0.6) (layer "F.Cu") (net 8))
 (segment (start 205 91) (end 207.08 91) (width 0.6) (layer "F.Cu") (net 8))
 (segment (start 194.5 97.5) (end 198.5 97.5) (width 0.6) (layer "F.Cu") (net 8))
 (segment (start 207.08 91) (end 210.5 87.58) (width 0.6) (layer "F.Cu") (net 8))
 (segment (start 182 92.057218) (end 183.594718 90.4625) (width 0.6) (layer "F.Cu") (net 8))
 (segment (start 197.1135 66.8865) (end 202.336098 66.8865) (width 0.6) (layer "F.Cu") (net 8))
 (segment (start 202.336098 66.8865) (end 203.04 67.590402) (width 0.6) (layer "F.Cu") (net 8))
 (segment (start 184.5 89.2) (end 183.5 88.2) (width 0.6) (layer "F.Cu") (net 11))
 (segment (start 183.5 88.2) (end 183.5 84.5) (width 0.6) (layer "F.Cu") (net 11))
 (segment (start 183.300169 89.2) (end 184.5 89.2) (width 0.6) (layer "F.Cu") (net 11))
 (segment (start 179.000168 93.5) (end 183.300169 89.2) (width 0.6) (layer "F.Cu") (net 11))
 (segment (start 173.5 93.5) (end 179.000168 93.5) (width 0.6) (layer "F.Cu") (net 11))
 (segment (start 183.5 84.5) (end 183.5 79) (width 0.6) (layer "F.Cu") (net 11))
 (segment (start 173.5 91.5) (end 177 91.5) (width 0.6) (layer "F.Cu") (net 12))
 (segment (start 184 66.5) (end 190 66.5) (width 0.6) (layer "F.Cu") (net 12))
 (segment (start 179 89.5) (end 179 71) (width 0.6) (layer "F.Cu") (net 12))
 (segment (start 183.5 66.5) (end 184 66.5) (width 0.6) (layer "F.Cu") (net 12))
 (segment (start 177 91.5) (end 179 89.5) (width 0.6) (layer "F.Cu") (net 12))
 (segment (start 179 71) (end 183.5 66.5) (width 0.6) (layer "F.Cu") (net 12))
 (segment (start 197 86) (end 199.8 86) (width 0.6) (layer "F.Cu") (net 15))
 (segment (start 199.8 86) (end 202.5 83.3) (width 0.6) (layer "F.Cu") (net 15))
 (segment (start 208.849 79.651) (end 208.849 79.071) (width 0.6) (layer "F.Cu") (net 6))
 (segment (start 200.5 78.5) (end 202.5 80.5) (width 0.6) (layer "F.Cu") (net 6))
 (segment (start 208 80.5) (end 208.849 79.651) (width 0.6) (layer "F.Cu") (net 6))
 (segment (start 202.5 80.5) (end 208 80.5) (width 0.6) (layer "F.Cu") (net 6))
 (segment (start 208.849 79.071) (end 210.5 77.42) (width 0.6) (layer "F.Cu") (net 6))
 (segment (start 200.5 68.5) (end 200.5 78.5) (width 0.6) (layer "F.Cu") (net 6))
 (segment (start 194.5 94.7) (end 198.8 94.7) (width 0.6) (layer "F.Cu") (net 9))
 (segment (start 198.8 94.7) (end 202.5 91) (width 0.6) (layer "F.Cu") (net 9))
 (segment (start 199.23 68.5) (end 194 73.73) (width 0.6) (layer "F.Cu") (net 5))
 (segment (start 194 73.73) (end 194 76) (width 0.6) (layer "F.Cu") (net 5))
 (segment (start 194 76) (end 200 82) (width 0.6) (layer "F.Cu") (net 5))
 (segment (start 208.46 82) (end 210.5 79.96) (width 0.6) (layer "F.Cu") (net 5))
 (segment (start 200 82) (end 208.46 82) (width 0.6) (layer "F.Cu") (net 5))
 (segment (start 201.77 61.325) (end 201.77 62.27) (width 0.6) (layer "F.Cu") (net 2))
 (segment (start 201.77 62.521648) (end 201.77 61.325) (width 0.6) (layer "F.Cu") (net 2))
 (segment (start 195.399 65.601) (end 198 65.601) (width 0.6) (layer "F.Cu") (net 2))
 (segment (start 201.77 62.521648) (end 201.77 62.5) (width 0.6) (layer "F.Cu") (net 2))
 (segment (start 198.690648 65.601) (end 201.77 62.521648) (width 0.6) (layer "F.Cu") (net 2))
 (segment (start 201.77 62.27) (end 208 68.5) (width 0.6) (layer "F.Cu") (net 2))
 (segment (start 185.5 79) (end 185.5 75.5) (width 0.6) (layer "F.Cu") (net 2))
 (segment (start 185.5 75.5) (end 194.5 66.5) (width 0.6) (layer "F.Cu") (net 2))
 (segment (start 198 65.601) (end 198.690648 65.601) (width 0.6) (layer "F.Cu") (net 2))
 (segment (start 208 69.84) (end 210.5 72.34) (width 0.6) (layer "F.Cu") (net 2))
 (segment (start 194.5 66.5) (end 195.399 65.601) (width 0.6) (layer "F.Cu") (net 2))
 (segment (start 208 68.5) (end 208 69.84) (width 0.6) (layer "F.Cu") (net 2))
 (segment (start 203 79.199) (end 207.16395 79.199) (width 0.6) (layer "F.Cu") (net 7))
 (segment (start 208.431475 76.948525) (end 210.5 74.88) (width 0.6) (layer "F.Cu") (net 7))
 (segment (start 208.431475 77.931475) (end 208.431475 76.948525) (width 0.6) (layer "F.Cu") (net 7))
 (segment (start 207.16395 79.199) (end 208.431475 77.931475) (width 0.6) (layer "F.Cu") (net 7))
 (segment (start 201.77 77.969) (end 203 79.199) (width 0.6) (layer "F.Cu") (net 7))
 (segment (start 201.77 68.5) (end 201.77 77.969) (width 0.6) (layer "F.Cu") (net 7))
 (segment (start 208.76 67.26) (end 210.5 67.26) (width 0.6) (layer "F.Cu") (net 1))
 (segment (start 208 66.285) (end 208 66.5) (width 0.6) (layer "F.Cu") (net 1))
 (segment (start 203.04 61.325) (end 208 66.285) (width 0.6) (layer "F.Cu") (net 1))
 (segment (start 208 66.5) (end 208.76 67.26) (width 0.6) (layer "F.Cu") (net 1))
 (segment (start 200.5 60.415402) (end 201.203902 59.7115) (width 0.6) (layer "F.Cu") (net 3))
 (segment (start 212.151 68.149) (end 210.5 69.8) (width 0.6) (layer "F.Cu") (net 3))
 (segment (start 212.151 64.036133) (end 212.151 68.149) (width 0.6) (layer "F.Cu") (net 3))
 (segment (start 201.203902 59.7115) (end 207.826367 59.7115) (width 0.6) (layer "F.Cu") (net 3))
 (segment (start 198.234598 64.5) (end 200.5 62.234598) (width 0.6) (layer "F.Cu") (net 3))
 (segment (start 207.826367 59.7115) (end 212.151 64.036133) (width 0.6) (layer "F.Cu") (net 3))
 (segment (start 200.5 61.325) (end 200.5 60.415402) (width 0.6) (layer "F.Cu") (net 3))
 (segment (start 200.5 62.234598) (end 200.5 61.325) (width 0.6) (layer "F.Cu") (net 3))
 (segment (start 184 64.5) (end 198.234598 64.5) (width 0.6) (layer "F.Cu") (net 3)))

